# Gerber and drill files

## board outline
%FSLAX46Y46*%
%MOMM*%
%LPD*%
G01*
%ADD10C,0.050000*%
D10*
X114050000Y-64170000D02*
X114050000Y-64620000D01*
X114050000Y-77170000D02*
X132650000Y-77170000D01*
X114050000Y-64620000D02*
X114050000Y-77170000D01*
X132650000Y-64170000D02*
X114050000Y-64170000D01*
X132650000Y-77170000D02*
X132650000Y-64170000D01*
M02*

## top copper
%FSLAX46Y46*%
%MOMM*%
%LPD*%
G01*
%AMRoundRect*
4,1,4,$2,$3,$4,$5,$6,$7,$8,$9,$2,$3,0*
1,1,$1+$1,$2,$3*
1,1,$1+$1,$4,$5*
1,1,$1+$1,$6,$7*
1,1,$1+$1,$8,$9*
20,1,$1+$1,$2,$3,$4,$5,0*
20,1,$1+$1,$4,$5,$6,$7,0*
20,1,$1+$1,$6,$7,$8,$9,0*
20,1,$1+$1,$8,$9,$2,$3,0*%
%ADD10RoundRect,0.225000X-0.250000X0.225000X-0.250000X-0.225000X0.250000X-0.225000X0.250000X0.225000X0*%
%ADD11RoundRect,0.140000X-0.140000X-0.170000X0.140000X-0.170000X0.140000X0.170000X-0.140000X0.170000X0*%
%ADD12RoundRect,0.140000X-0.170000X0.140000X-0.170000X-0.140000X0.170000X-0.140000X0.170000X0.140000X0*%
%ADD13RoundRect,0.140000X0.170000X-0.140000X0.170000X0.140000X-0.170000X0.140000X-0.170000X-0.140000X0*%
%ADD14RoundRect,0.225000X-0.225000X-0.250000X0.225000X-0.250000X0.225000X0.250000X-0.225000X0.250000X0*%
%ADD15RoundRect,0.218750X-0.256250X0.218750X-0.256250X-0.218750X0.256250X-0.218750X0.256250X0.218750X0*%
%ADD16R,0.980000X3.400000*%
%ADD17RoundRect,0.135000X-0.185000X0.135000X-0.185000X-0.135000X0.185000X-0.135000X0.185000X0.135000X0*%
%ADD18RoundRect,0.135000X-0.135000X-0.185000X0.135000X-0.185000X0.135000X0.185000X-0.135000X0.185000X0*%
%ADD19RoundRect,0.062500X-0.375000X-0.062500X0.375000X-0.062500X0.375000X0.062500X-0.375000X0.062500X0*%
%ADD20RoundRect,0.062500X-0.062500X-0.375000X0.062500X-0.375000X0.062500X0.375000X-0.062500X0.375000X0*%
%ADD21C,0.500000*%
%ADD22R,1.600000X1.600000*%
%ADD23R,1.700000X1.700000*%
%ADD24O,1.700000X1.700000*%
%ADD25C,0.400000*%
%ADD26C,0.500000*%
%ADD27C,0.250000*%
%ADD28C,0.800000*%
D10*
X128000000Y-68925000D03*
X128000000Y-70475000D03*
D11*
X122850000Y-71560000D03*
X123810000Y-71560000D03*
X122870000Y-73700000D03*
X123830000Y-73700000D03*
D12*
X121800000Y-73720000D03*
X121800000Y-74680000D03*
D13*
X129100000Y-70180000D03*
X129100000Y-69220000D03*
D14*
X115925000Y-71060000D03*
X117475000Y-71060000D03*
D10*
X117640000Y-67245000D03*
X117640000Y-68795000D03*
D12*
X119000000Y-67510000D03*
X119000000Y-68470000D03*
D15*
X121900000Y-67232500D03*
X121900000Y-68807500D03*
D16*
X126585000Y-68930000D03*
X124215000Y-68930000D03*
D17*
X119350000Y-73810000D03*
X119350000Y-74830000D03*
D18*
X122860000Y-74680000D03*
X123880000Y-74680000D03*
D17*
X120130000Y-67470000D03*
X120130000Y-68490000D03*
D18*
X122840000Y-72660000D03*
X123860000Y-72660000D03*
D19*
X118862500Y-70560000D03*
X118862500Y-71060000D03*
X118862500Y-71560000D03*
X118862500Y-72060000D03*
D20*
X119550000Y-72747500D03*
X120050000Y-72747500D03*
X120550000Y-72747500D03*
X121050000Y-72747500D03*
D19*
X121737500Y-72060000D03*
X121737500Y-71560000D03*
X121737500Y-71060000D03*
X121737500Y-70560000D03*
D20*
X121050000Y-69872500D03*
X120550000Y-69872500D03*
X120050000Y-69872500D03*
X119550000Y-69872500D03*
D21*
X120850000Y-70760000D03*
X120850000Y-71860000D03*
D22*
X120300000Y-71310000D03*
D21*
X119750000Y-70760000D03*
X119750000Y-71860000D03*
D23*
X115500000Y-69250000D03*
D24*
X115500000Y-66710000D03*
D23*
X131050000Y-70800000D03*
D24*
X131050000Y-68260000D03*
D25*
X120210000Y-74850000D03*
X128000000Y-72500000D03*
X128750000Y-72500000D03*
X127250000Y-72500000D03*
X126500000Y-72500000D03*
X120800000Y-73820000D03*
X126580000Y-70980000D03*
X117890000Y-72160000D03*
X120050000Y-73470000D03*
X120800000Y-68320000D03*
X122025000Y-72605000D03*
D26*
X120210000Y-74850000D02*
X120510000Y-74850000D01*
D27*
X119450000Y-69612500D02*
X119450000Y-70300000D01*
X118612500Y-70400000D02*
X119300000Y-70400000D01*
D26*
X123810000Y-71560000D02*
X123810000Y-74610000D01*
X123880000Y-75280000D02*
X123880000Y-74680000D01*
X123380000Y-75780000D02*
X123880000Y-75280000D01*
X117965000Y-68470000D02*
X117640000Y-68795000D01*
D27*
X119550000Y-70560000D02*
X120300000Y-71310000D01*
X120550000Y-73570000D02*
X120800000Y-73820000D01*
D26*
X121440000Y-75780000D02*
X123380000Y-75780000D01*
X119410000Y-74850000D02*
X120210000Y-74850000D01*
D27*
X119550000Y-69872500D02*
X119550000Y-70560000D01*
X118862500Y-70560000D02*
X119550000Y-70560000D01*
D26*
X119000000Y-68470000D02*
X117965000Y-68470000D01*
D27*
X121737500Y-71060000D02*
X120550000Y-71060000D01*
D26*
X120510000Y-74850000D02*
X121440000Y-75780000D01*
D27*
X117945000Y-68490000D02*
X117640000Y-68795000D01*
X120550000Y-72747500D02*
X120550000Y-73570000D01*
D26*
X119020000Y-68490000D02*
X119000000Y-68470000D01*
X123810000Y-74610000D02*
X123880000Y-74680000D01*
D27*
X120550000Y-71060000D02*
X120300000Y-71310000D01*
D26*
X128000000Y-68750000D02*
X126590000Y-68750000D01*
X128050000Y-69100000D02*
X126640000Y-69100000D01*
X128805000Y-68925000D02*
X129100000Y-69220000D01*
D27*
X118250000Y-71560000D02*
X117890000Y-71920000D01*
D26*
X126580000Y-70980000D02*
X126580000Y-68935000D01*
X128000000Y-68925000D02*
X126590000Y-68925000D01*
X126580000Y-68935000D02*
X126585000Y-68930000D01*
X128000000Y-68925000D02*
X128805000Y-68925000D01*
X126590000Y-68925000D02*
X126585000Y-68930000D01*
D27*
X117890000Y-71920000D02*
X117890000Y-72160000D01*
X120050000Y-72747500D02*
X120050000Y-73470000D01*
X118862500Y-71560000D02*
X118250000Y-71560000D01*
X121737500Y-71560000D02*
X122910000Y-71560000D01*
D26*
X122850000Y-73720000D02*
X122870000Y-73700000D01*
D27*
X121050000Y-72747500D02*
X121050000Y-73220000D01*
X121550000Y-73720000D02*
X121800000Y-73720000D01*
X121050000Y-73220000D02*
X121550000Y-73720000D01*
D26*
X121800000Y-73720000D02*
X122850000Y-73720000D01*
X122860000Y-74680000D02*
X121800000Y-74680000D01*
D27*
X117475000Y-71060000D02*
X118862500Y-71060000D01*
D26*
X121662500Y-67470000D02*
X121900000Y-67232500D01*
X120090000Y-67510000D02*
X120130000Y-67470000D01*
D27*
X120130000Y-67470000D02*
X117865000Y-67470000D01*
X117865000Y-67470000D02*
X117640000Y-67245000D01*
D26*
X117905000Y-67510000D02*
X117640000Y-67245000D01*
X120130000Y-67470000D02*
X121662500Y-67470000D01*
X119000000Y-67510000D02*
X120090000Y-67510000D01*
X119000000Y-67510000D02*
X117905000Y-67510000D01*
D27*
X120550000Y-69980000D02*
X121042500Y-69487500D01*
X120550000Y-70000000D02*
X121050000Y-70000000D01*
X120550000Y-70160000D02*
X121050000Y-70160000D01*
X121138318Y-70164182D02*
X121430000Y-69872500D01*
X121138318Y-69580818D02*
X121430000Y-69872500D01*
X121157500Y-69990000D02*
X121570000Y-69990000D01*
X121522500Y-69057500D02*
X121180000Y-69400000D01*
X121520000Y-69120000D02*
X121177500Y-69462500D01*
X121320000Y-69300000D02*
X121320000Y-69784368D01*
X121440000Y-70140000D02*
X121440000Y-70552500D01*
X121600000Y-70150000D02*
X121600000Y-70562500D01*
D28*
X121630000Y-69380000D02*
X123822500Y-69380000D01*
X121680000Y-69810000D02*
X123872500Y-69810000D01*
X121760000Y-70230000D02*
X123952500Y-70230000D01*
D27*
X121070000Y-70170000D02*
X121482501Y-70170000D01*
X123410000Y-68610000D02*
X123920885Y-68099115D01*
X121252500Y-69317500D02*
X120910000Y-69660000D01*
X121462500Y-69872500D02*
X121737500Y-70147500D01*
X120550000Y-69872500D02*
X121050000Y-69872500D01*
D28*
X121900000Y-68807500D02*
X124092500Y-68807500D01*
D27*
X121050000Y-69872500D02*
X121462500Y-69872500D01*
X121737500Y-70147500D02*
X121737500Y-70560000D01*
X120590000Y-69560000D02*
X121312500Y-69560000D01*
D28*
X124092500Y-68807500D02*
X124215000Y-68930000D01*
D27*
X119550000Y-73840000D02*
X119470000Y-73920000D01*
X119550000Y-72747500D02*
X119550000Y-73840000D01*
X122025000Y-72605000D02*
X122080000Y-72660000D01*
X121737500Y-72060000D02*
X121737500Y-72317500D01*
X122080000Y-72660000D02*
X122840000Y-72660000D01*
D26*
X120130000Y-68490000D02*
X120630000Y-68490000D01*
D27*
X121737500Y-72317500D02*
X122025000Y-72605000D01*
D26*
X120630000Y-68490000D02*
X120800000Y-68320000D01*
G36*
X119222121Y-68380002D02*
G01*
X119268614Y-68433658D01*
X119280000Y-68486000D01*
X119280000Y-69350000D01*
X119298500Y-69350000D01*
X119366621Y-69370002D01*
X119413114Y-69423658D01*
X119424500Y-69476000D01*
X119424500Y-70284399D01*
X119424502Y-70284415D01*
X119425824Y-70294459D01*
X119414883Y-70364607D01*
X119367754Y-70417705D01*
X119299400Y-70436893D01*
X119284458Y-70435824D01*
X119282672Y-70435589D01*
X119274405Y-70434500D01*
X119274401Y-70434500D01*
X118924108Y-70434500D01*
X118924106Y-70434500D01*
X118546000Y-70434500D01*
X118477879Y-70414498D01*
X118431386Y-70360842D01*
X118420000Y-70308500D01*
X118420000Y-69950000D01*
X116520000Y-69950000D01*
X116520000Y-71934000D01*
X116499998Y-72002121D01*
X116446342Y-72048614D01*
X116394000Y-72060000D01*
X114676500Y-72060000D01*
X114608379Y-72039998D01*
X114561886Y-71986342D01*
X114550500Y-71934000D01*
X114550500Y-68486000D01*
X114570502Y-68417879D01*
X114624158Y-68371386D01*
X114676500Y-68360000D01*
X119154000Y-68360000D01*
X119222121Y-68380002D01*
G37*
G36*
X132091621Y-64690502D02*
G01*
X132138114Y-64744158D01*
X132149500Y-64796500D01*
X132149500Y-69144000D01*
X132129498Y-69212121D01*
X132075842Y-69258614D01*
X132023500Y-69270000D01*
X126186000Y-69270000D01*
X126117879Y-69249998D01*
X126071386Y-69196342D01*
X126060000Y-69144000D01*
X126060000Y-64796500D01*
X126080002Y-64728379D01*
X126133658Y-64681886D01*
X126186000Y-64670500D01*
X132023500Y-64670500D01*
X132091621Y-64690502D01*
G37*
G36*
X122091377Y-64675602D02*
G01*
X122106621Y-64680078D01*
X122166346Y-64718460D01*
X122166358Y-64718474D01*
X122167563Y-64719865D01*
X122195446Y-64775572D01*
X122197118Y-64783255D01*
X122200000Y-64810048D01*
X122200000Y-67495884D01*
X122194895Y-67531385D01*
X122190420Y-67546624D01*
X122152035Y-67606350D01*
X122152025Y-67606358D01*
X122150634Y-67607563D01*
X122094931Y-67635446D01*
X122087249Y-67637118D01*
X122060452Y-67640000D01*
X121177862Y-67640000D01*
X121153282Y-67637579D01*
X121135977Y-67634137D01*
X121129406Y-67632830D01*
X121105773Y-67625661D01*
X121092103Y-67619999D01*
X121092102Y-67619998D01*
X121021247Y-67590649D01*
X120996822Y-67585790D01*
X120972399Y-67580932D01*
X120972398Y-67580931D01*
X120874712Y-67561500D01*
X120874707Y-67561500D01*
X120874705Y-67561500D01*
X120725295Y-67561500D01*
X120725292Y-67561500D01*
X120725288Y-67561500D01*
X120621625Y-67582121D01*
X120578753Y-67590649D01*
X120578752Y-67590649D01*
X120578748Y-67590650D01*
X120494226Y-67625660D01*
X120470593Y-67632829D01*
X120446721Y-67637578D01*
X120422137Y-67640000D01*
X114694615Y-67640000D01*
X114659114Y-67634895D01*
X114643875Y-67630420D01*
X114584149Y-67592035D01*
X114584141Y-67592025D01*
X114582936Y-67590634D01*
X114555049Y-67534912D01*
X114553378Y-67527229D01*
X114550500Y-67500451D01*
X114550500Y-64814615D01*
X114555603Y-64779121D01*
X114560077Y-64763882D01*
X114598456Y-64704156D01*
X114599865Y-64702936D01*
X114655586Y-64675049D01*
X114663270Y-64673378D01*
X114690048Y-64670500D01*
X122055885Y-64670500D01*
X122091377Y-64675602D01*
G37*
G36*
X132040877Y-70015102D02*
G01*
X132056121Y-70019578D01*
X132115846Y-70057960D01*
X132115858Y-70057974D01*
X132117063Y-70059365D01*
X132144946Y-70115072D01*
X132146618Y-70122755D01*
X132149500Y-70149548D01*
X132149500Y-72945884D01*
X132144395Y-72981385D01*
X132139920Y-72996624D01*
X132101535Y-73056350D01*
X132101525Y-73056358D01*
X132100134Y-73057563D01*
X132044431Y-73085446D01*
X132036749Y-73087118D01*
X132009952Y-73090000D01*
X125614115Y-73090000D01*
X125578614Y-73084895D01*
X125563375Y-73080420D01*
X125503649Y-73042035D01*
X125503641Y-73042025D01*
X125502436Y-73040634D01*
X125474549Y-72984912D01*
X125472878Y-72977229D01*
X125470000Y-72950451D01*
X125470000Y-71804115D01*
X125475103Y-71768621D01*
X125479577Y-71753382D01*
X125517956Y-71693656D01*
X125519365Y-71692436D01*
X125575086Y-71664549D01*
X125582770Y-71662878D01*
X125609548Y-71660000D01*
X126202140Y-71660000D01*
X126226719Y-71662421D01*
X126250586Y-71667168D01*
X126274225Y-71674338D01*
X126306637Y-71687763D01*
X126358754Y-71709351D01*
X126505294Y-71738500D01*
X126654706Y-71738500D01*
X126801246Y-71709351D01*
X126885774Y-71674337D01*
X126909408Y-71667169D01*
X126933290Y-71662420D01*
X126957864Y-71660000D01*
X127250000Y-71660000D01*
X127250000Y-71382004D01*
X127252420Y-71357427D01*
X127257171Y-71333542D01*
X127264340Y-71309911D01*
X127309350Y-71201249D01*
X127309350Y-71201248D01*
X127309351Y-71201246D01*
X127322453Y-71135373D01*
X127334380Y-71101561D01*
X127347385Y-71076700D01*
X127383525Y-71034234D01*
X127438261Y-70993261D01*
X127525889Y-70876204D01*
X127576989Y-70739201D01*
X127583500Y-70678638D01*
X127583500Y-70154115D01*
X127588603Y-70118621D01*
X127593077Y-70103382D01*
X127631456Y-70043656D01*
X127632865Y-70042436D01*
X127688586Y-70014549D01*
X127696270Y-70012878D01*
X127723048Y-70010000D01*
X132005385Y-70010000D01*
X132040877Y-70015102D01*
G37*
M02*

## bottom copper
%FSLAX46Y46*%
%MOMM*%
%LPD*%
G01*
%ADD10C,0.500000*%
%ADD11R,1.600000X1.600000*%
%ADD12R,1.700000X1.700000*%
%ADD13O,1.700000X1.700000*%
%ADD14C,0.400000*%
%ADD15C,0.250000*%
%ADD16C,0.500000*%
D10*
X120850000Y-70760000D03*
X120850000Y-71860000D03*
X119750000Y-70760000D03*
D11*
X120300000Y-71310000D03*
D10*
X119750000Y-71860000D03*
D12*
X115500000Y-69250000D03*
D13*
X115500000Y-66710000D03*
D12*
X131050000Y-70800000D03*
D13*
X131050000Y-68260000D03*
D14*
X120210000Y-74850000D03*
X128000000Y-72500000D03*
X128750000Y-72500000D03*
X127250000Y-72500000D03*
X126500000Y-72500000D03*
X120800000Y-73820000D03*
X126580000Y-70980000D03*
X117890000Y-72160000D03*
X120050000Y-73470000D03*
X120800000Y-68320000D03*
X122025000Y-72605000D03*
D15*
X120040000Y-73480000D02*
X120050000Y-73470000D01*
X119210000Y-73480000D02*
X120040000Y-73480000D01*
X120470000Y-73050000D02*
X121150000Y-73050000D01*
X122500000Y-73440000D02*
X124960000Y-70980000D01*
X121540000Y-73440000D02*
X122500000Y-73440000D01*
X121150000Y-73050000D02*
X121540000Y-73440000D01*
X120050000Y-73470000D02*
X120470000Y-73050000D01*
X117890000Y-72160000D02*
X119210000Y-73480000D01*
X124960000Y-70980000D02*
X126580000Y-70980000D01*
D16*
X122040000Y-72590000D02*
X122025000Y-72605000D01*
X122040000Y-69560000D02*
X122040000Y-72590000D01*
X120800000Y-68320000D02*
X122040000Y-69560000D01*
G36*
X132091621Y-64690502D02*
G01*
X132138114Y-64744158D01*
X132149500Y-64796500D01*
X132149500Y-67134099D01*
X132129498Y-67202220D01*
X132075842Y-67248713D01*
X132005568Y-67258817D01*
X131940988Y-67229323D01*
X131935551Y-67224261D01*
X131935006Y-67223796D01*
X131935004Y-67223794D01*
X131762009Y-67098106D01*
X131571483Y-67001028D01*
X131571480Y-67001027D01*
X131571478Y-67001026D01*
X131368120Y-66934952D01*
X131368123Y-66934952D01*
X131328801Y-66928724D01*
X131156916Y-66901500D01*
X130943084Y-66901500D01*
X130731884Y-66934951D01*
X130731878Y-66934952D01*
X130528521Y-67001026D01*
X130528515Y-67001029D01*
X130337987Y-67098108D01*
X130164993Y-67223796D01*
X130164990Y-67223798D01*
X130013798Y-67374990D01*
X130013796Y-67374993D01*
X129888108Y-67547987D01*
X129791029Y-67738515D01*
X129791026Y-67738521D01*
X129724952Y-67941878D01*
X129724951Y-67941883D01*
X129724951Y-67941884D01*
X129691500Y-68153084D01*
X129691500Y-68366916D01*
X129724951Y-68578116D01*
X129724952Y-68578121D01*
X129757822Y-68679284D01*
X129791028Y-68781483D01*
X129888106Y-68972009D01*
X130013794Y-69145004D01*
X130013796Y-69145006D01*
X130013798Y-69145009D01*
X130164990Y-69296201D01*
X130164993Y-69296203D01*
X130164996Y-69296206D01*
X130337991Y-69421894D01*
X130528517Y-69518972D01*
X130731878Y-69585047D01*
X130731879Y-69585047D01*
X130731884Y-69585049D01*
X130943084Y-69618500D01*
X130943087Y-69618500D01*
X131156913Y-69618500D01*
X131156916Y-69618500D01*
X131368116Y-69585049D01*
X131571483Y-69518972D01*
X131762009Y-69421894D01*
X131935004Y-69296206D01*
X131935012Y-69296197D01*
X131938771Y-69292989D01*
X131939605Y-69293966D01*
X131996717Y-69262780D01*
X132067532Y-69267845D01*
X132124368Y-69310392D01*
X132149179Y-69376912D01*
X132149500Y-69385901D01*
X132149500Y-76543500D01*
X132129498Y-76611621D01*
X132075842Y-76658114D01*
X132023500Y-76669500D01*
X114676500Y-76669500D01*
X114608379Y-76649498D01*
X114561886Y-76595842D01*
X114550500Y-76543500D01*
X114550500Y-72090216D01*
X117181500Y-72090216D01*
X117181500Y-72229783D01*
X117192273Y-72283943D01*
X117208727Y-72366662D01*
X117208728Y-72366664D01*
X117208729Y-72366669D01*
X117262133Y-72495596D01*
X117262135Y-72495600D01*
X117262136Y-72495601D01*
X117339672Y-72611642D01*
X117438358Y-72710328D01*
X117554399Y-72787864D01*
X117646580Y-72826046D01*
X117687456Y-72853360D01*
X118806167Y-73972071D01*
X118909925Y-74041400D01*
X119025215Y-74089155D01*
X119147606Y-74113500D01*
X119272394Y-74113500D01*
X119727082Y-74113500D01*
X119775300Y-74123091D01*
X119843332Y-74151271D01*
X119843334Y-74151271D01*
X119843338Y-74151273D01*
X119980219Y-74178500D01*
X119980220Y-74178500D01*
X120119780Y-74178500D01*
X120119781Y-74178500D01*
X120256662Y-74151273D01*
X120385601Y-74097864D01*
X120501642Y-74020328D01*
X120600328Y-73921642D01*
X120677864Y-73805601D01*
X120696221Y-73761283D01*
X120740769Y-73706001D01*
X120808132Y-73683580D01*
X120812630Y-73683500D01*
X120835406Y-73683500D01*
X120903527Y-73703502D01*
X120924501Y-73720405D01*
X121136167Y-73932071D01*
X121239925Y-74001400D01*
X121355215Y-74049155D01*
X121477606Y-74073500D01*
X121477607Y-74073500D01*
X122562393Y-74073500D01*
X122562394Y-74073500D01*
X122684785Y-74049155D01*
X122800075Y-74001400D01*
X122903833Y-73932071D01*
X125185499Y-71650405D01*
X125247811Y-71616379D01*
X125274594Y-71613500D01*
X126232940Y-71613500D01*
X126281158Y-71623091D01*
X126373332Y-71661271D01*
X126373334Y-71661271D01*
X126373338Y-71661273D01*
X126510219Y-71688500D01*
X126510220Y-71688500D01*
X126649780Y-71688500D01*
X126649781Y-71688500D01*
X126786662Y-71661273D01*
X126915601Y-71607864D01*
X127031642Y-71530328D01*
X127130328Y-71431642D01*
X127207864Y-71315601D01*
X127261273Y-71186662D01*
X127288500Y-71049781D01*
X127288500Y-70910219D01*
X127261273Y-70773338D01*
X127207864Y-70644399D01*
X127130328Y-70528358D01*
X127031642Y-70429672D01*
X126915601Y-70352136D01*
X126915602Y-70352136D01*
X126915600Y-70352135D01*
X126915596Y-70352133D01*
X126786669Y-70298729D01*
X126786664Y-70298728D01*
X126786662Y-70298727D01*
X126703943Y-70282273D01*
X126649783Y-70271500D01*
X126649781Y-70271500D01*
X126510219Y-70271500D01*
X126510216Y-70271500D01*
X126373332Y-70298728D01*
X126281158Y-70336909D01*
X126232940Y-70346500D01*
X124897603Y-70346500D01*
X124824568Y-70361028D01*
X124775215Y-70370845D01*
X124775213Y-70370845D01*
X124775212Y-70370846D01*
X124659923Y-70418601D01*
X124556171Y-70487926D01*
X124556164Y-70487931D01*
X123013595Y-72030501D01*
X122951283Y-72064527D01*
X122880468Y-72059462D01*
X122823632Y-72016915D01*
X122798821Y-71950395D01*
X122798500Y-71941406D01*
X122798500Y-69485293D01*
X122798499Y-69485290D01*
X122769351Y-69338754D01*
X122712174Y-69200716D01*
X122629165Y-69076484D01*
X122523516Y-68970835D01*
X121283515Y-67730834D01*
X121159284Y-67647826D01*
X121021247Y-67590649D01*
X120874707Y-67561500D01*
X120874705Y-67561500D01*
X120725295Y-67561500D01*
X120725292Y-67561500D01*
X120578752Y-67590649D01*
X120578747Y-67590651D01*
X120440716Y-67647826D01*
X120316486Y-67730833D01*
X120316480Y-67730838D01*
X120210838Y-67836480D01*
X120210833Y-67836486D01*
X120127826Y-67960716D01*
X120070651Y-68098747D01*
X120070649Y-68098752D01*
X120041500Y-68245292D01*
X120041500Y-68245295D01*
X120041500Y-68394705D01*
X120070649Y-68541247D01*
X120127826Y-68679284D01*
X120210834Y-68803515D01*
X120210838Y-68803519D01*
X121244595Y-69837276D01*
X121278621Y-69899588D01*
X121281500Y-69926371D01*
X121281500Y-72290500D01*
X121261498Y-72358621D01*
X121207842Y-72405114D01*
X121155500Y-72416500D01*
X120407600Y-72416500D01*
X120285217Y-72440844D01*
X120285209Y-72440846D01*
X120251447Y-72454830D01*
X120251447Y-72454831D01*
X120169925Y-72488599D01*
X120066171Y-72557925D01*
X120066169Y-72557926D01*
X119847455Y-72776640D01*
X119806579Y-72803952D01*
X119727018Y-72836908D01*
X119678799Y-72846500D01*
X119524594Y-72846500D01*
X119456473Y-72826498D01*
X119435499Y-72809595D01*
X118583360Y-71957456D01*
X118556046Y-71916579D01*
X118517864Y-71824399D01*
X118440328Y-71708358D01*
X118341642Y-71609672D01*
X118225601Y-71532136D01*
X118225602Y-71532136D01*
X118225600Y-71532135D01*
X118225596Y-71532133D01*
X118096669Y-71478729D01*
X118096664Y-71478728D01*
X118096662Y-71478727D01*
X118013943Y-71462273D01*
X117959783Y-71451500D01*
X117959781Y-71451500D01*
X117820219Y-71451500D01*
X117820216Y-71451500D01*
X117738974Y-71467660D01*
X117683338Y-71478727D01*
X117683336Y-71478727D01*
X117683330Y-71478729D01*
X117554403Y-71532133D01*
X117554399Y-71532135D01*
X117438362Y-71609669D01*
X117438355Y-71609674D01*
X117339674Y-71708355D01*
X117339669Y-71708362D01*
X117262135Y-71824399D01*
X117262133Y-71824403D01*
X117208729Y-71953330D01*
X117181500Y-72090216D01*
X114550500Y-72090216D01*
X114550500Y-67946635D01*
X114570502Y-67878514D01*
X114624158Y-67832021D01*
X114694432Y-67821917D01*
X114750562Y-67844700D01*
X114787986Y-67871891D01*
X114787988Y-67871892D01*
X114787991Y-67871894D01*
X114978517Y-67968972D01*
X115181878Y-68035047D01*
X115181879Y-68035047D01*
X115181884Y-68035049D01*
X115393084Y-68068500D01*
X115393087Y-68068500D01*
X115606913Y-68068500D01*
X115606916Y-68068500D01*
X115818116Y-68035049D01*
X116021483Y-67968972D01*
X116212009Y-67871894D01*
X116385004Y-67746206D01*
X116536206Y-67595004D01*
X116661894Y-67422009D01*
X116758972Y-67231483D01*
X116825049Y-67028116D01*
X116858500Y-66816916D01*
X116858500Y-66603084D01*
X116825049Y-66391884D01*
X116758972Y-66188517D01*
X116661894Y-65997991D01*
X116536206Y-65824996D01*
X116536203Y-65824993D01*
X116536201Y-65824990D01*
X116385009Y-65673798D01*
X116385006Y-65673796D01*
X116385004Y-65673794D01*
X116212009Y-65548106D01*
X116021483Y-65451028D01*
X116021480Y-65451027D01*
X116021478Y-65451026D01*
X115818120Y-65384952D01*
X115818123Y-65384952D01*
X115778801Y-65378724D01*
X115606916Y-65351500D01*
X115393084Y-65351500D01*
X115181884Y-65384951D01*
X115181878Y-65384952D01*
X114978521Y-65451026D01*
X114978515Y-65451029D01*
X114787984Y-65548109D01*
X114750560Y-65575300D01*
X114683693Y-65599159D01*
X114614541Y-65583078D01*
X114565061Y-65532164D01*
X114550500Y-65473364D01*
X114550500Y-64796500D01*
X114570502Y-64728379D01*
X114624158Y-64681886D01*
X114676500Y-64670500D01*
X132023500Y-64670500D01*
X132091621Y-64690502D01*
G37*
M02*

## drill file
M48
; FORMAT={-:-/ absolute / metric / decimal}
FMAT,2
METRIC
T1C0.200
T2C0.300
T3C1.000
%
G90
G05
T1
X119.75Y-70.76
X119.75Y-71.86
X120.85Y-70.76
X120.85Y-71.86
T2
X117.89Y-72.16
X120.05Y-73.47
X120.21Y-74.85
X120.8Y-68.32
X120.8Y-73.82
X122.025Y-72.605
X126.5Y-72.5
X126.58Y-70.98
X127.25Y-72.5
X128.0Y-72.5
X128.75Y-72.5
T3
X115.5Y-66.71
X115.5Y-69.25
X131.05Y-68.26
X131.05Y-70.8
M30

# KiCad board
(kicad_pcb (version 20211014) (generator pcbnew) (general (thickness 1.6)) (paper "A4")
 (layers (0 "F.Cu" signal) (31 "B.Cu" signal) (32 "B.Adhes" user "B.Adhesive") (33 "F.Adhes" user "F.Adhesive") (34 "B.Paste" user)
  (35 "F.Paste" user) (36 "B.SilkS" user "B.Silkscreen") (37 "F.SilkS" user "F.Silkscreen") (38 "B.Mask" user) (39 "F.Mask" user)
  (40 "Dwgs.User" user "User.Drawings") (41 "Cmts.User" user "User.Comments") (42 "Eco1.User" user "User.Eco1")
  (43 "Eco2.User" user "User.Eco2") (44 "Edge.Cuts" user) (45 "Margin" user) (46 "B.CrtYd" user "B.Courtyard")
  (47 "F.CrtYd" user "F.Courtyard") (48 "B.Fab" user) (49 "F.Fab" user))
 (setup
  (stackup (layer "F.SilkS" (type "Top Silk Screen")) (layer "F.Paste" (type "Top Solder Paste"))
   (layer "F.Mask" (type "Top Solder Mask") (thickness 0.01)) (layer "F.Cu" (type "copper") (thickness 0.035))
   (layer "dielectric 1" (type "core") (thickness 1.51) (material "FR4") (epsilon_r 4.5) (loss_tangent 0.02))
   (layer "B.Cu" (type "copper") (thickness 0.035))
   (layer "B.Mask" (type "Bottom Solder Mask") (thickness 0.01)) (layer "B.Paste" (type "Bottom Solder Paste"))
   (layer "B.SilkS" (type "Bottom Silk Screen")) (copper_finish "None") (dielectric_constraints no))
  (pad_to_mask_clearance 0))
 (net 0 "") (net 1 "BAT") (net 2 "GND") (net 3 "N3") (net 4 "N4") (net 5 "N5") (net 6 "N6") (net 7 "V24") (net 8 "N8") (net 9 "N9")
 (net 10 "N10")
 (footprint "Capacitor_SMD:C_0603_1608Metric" (layer "F.Cu") (at 128 69.7 -90)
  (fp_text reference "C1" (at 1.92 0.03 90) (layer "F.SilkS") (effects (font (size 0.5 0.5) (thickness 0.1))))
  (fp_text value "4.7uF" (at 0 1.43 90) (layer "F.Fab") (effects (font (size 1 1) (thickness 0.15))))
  (pad "1" smd roundrect locked (at -0.775 0 270) (size 0.9 0.95) (layers "F.Cu" "F.Paste" "F.Mask") (roundrect_rratio 0.25) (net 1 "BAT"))
  (pad "2" smd roundrect locked (at 0.775 0 270) (size 0.9 0.95) (layers "F.Cu" "F.Paste" "F.Mask") (roundrect_rratio 0.25) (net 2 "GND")))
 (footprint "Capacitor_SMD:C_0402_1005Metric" (layer "F.Cu") (at 123.33 71.56)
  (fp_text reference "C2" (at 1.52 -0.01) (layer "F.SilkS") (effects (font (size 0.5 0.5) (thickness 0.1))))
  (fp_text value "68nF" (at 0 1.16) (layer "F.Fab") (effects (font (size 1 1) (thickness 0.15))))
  (pad "1" smd roundrect locked (at -0.48 0) (size 0.56 0.62) (layers "F.Cu" "F.Paste" "F.Mask") (roundrect_rratio 0.25) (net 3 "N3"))
  (pad "2" smd roundrect locked (at 0.48 0) (size 0.56 0.62) (layers "F.Cu" "F.Paste" "F.Mask") (roundrect_rratio 0.25) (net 2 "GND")))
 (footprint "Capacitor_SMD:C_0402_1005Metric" (layer "F.Cu") (at 123.35 73.7)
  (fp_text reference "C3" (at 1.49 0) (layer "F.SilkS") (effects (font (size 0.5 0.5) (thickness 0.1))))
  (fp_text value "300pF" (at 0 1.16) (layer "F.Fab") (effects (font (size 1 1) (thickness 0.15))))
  (pad "1" smd roundrect locked (at -0.48 0) (size 0.56 0.62) (layers "F.Cu" "F.Paste" "F.Mask") (roundrect_rratio 0.25) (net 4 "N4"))
  (pad "2" smd roundrect locked (at 0.48 0) (size 0.56 0.62) (layers "F.Cu" "F.Paste" "F.Mask") (roundrect_rratio 0.25) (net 2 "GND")))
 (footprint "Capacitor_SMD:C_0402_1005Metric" (layer "F.Cu") (at 121.8 74.2 -90)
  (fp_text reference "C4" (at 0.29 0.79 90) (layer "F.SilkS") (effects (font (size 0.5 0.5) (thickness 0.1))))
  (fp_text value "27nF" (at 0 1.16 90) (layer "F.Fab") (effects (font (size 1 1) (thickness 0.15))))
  (pad "1" smd roundrect locked (at -0.48 0 270) (size 0.56 0.62) (layers "F.Cu" "F.Paste" "F.Mask") (roundrect_rratio 0.25) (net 4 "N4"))
  (pad "2" smd roundrect locked (at 0.48 0 270) (size 0.56 0.62) (layers "F.Cu" "F.Paste" "F.Mask") (roundrect_rratio 0.25) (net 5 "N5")))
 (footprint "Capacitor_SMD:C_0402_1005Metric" (layer "F.Cu") (at 129.1 69.7 90)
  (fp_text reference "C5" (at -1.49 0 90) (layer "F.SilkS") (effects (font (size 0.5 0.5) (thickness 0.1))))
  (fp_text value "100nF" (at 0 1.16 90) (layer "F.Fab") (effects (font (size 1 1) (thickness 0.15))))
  (pad "1" smd roundrect locked (at -0.48 0 90) (size 0.56 0.62) (layers "F.Cu" "F.Paste" "F.Mask") (roundrect_rratio 0.25) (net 2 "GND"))
  (pad "2" smd roundrect locked (at 0.48 0 90) (size 0.56 0.62) (layers "F.Cu" "F.Paste" "F.Mask") (roundrect_rratio 0.25) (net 1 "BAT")))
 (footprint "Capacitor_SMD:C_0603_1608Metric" (layer "F.Cu") (at 116.7 71.06)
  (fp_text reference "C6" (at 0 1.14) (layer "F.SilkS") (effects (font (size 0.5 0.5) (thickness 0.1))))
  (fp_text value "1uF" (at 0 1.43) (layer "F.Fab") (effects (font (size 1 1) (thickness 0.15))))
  (pad "1" smd roundrect locked (at -0.775 0) (size 0.9 0.95) (layers "F.Cu" "F.Paste" "F.Mask") (roundrect_rratio 0.25) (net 2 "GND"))
  (pad "2" smd roundrect locked (at 0.775 0) (size 0.9 0.95) (layers "F.Cu" "F.Paste" "F.Mask") (roundrect_rratio 0.25) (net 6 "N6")))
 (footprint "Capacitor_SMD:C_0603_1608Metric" (layer "F.Cu") (at 117.64 68.02 -90)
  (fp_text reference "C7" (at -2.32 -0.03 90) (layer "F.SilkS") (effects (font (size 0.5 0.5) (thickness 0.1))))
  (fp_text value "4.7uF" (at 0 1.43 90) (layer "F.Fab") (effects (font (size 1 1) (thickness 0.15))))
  (pad "1" smd roundrect locked (at -0.775 0 270) (size 0.9 0.95) (layers "F.Cu" "F.Paste" "F.Mask") (roundrect_rratio 0.25) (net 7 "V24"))
  (pad "2" smd roundrect locked (at 0.775 0 270) (size 0.9 0.95) (layers "F.Cu" "F.Paste" "F.Mask") (roundrect_rratio 0.25) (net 2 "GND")))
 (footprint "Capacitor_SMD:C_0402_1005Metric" (layer "F.Cu") (at 119 67.99 -90)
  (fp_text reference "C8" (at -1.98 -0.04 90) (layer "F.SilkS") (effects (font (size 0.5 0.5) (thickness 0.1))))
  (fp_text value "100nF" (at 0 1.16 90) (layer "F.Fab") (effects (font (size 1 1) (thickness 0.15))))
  (pad "1" smd roundrect locked (at -0.48 0 270) (size 0.56 0.62) (layers "F.Cu" "F.Paste" "F.Mask") (roundrect_rratio 0.25) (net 7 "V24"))
  (pad "2" smd roundrect locked (at 0.48 0 270) (size 0.56 0.62) (layers "F.Cu" "F.Paste" "F.Mask") (roundrect_rratio 0.25) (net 2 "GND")))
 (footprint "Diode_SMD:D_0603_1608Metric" (layer "F.Cu") (at 121.9 68.02 -90)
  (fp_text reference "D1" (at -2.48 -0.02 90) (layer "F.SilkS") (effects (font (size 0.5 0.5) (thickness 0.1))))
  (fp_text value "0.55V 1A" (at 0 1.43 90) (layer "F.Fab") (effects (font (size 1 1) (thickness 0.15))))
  (pad "1" smd roundrect locked (at -0.7875 0 270) (size 0.875 0.95) (layers "F.Cu" "F.Paste" "F.Mask") (roundrect_rratio 0.25)
   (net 7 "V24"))
  (pad "2" smd roundrect locked (at 0.7875 0 270) (size 0.875 0.95) (layers "F.Cu" "F.Paste" "F.Mask") (roundrect_rratio 0.25) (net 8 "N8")))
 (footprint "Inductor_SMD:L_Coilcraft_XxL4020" (layer "F.Cu") (at 125.4 68.93 180)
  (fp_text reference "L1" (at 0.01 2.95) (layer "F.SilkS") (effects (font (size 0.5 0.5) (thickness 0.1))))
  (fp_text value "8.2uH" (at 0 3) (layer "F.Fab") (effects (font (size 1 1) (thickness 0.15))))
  (pad "1" smd rect locked (at -1.185 0 180) (size 0.98 3.4) (layers "F.Cu" "F.Paste" "F.Mask") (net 1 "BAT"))
  (pad "2" smd rect locked (at 1.185 0 180) (size 0.98 3.4) (layers "F.Cu" "F.Paste" "F.Mask") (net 8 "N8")))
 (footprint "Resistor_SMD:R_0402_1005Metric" (layer "F.Cu") (at 119.35 74.32 -90)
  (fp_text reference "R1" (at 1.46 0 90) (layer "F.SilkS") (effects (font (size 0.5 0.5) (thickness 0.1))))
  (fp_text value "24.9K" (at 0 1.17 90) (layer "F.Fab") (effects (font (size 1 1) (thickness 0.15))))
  (pad "1" smd roundrect locked (at -0.51 0 270) (size 0.54 0.64) (layers "F.Cu" "F.Paste" "F.Mask") (roundrect_rratio 0.25) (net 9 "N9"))
  (pad "2" smd roundrect locked (at 0.51 0 270) (size 0.54 0.64) (layers "F.Cu" "F.Paste" "F.Mask") (roundrect_rratio 0.25) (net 2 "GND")))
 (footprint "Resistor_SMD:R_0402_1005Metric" (layer "F.Cu") (at 123.37 74.68)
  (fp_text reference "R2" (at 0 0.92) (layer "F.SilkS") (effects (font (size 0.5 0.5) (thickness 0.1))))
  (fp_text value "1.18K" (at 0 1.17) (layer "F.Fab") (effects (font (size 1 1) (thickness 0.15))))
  (pad "1" smd roundrect locked (at -0.51 0) (size 0.54 0.64) (layers "F.Cu" "F.Paste" "F.Mask") (roundrect_rratio 0.25) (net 5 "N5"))
  (pad "2" smd roundrect locked (at 0.51 0) (size 0.54 0.64) (layers "F.Cu" "F.Paste" "F.Mask") (roundrect_rratio 0.25) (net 2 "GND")))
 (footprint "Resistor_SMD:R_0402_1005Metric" (layer "F.Cu") (at 120.13 67.98 -90)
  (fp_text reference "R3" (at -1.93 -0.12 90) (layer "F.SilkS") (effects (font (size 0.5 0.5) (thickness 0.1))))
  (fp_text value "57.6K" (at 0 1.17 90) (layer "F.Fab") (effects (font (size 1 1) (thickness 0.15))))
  (pad "1" smd roundrect locked (at -0.51 0 270) (size 0.54 0.64) (layers "F.Cu" "F.Paste" "F.Mask") (roundrect_rratio 0.25) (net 7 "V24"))
  (pad "2" smd roundrect locked (at 0.51 0 270) (size 0.54 0.64) (layers "F.Cu" "F.Paste" "F.Mask") (roundrect_rratio 0.25) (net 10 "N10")))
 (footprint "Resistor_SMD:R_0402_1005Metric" (layer "F.Cu") (at 123.35 72.66)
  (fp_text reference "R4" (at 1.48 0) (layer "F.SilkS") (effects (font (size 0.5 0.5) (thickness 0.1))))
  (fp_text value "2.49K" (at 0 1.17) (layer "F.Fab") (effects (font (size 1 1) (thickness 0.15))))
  (pad "1" smd roundrect locked (at -0.51 0) (size 0.54 0.64) (layers "F.Cu" "F.Paste" "F.Mask") (roundrect_rratio 0.25) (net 10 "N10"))
  (pad "2" smd roundrect locked (at 0.51 0) (size 0.54 0.64) (layers "F.Cu" "F.Paste" "F.Mask") (roundrect_rratio 0.25) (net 2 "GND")))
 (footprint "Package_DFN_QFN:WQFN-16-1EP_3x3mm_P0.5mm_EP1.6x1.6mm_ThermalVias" (layer "F.Cu") (at 120.3 71.31)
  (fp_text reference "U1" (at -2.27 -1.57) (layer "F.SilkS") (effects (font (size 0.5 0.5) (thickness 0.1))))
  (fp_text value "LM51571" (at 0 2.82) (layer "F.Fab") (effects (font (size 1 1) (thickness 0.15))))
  (pad "" smd roundrect locked (at 0.4 0.4) (size 0.69 0.69) (layers "F.Paste") (roundrect_rratio 0.25))
  (pad "" smd roundrect locked (at 0.4 -0.4) (size 0.69 0.69) (layers "F.Paste") (roundrect_rratio 0.25))
  (pad "" smd roundrect locked (at -0.4 0.4) (size 0.69 0.69) (layers "F.Paste") (roundrect_rratio 0.25))
  (pad "" smd roundrect locked (at -0.4 -0.4) (size 0.69 0.69) (layers "F.Paste") (roundrect_rratio 0.25))
  (pad "1" smd roundrect locked (at -1.4375 -0.75) (size 0.875 0.25) (layers "F.Cu" "F.Paste" "F.Mask") (roundrect_rratio 0.25)
   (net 2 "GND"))
  (pad "2" smd roundrect locked (at -1.4375 -0.25) (size 0.875 0.25) (layers "F.Cu" "F.Paste" "F.Mask") (roundrect_rratio 0.25) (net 6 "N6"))
  (pad "3" smd roundrect locked (at -1.4375 0.25) (size 0.875 0.25) (layers "F.Cu" "F.Paste" "F.Mask") (roundrect_rratio 0.25) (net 1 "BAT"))
  (pad "4" smd roundrect locked (at -1.4375 0.75) (size 0.875 0.25) (layers "F.Cu" "F.Paste" "F.Mask") (roundrect_rratio 0.25))
  (pad "5" smd roundrect locked (at -0.75 1.4375) (size 0.25 0.875) (layers "F.Cu" "F.Paste" "F.Mask") (roundrect_rratio 0.25) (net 9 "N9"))
  (pad "6" smd roundrect locked (at -0.25 1.4375) (size 0.25 0.875) (layers "F.Cu" "F.Paste" "F.Mask") (roundrect_rratio 0.25) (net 1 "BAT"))
  (pad "7" smd roundrect locked (at 0.25 1.4375) (size 0.25 0.875) (layers "F.Cu" "F.Paste" "F.Mask") (roundrect_rratio 0.25) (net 2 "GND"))
  (pad "8" smd roundrect locked (at 0.75 1.4375) (size 0.25 0.875) (layers "F.Cu" "F.Paste" "F.Mask") (roundrect_rratio 0.25) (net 4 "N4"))
  (pad "9" smd roundrect locked (at 1.4375 0.75) (size 0.875 0.25) (layers "F.Cu" "F.Paste" "F.Mask") (roundrect_rratio 0.25) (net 10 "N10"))
  (pad "10" smd roundrect locked (at 1.4375 0.25) (size 0.875 0.25) (layers "F.Cu" "F.Paste" "F.Mask") (roundrect_rratio 0.25) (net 3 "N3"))
  (pad "11" smd roundrect locked (at 1.4375 -0.25) (size 0.875 0.25) (layers "F.Cu" "F.Paste" "F.Mask") (roundrect_rratio 0.25)
   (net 2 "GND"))
  (pad "12" smd roundrect locked (at 1.4375 -0.75) (size 0.875 0.25) (layers "F.Cu" "F.Paste" "F.Mask") (roundrect_rratio 0.25) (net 8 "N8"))
  (pad "13" smd roundrect locked (at 0.75 -1.4375) (size 0.25 0.875) (layers "F.Cu" "F.Paste" "F.Mask") (roundrect_rratio 0.25) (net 8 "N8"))
  (pad "14" smd roundrect locked (at 0.25 -1.4375) (size 0.25 0.875) (layers "F.Cu" "F.Paste" "F.Mask") (roundrect_rratio 0.25) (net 8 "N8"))
  (pad "15" smd roundrect locked (at -0.25 -1.4375) (size 0.25 0.875) (layers "F.Cu" "F.Paste" "F.Mask") (roundrect_rratio 0.25))
  (pad "16" smd roundrect locked (at -0.75 -1.4375) (size 0.25 0.875) (layers "F.Cu" "F.Paste" "F.Mask") (roundrect_rratio 0.25)
   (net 2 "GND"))
  (pad "17" thru_hole circle locked (at 0.55 -0.55) (size 0.5 0.5) (drill 0.2) (layers *.Cu) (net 2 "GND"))
  (pad "17" thru_hole circle locked (at 0.55 0.55) (size 0.5 0.5) (drill 0.2) (layers *.Cu) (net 2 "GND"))
  (pad "17" smd rect locked (at 0 0) (size 1.6 1.6) (layers "F.Cu" "F.Mask") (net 2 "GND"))
  (pad "17" thru_hole circle locked (at -0.55 -0.55) (size 0.5 0.5) (drill 0.2) (layers *.Cu) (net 2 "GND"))
  (pad "17" smd rect locked (at 0 0) (size 1.6 1.6) (layers "B.Cu") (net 2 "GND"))
  (pad "17" thru_hole circle locked (at -0.55 0.55) (size 0.5 0.5) (drill 0.2) (layers *.Cu) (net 2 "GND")))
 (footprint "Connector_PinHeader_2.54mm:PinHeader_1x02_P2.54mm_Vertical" (layer "F.Cu") (at 115.5 69.25 180)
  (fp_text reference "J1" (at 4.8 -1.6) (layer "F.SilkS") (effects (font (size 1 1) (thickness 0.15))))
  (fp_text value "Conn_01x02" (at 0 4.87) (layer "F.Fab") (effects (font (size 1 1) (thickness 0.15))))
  (pad "1" thru_hole rect locked (at 0 0 180) (size 1.7 1.7) (drill 1) (layers *.Cu *.Mask) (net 2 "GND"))
  (pad "2" thru_hole oval locked (at 0 2.54 180) (size 1.7 1.7) (drill 1) (layers *.Cu *.Mask) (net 7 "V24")))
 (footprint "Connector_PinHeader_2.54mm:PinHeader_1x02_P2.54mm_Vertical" (layer "F.Cu") (at 131.05 70.8 180)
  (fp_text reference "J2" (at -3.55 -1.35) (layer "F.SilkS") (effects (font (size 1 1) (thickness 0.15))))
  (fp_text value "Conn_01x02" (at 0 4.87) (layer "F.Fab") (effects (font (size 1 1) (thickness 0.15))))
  (pad "1" thru_hole rect locked (at 0 0 180) (size 1.7 1.7) (drill 1) (layers *.Cu *.Mask) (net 2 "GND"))
  (pad "2" thru_hole oval locked (at 0 2.54 180) (size 1.7 1.7) (drill 1) (layers *.Cu *.Mask) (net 1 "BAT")))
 (gr_line (start 114.05 64.17) (end 114.05 64.62) (layer "Edge.Cuts") (width 0.05))
 (gr_line (start 114.05 77.17) (end 132.65 77.17) (layer "Edge.Cuts") (width 0.05))
 (gr_line (start 114.05 64.62) (end 114.05 77.17) (layer "Edge.Cuts") (width 0.05))
 (gr_line (start 132.65 64.17) (end 114.05 64.17) (layer "Edge.Cuts") (width 0.05))
 (gr_line (start 132.65 77.17) (end 132.65 64.17) (layer "Edge.Cuts") (width 0.05))
 (segment (start 120.21 74.85) (end 120.51 74.85) (width 0.5) (layer "F.Cu") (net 2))
 (segment (start 119.45 69.6125) (end 119.45 70.3) (width 0.25) (layer "F.Cu") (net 2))
 (segment (start 118.6125 70.4) (end 119.3 70.4) (width 0.25) (layer "F.Cu") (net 2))
 (segment (start 123.81 71.56) (end 123.81 74.61) (width 0.5) (layer "F.Cu") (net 2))
 (segment (start 123.88 75.28) (end 123.88 74.68) (width 0.5) (layer "F.Cu") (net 2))
 (segment (start 123.38 75.78) (end 123.88 75.28) (width 0.5) (layer "F.Cu") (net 2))
 (segment (start 117.965 68.47) (end 117.64 68.795) (width 0.5) (layer "F.Cu") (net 2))
 (segment (start 119.55 70.56) (end 120.3 71.31) (width 0.25) (layer "F.Cu") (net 2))
 (segment (start 120.55 73.57) (end 120.8 73.82) (width 0.25) (layer "F.Cu") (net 2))
 (segment (start 121.44 75.78) (end 123.38 75.78) (width 0.5) (layer "F.Cu") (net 2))
 (segment (start 119.41 74.85) (end 120.21 74.85) (width 0.5) (layer "F.Cu") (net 2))
 (segment (start 119.55 69.8725) (end 119.55 70.56) (width 0.25) (layer "F.Cu") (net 2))
 (segment (start 118.8625 70.56) (end 119.55 70.56) (width 0.25) (layer "F.Cu") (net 2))
 (segment (start 119 68.47) (end 117.965 68.47) (width 0.5) (layer "F.Cu") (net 2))
 (segment (start 121.7375 71.06) (end 120.55 71.06) (width 0.25) (layer "F.Cu") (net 2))
 (segment (start 120.51 74.85) (end 121.44 75.78) (width 0.5) (layer "F.Cu") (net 2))
 (segment (start 117.945 68.49) (end 117.64 68.795) (width 0.25) (layer "F.Cu") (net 2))
 (segment (start 120.55 72.7475) (end 120.55 73.57) (width 0.25) (layer "F.Cu") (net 2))
 (segment (start 119.02 68.49) (end 119 68.47) (width 0.5) (layer "F.Cu") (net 2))
 (segment (start 123.81 74.61) (end 123.88 74.68) (width 0.5) (layer "F.Cu") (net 2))
 (segment (start 120.55 71.06) (end 120.3 71.31) (width 0.25) (layer "F.Cu") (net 2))
 (via (at 120.21 74.85) (size 0.4) (drill 0.3) (layers "F.Cu" "B.Cu") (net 2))
 (via (at 128 72.5) (size 0.4) (drill 0.3) (layers "F.Cu" "B.Cu") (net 2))
 (via (at 128.75 72.5) (size 0.4) (drill 0.3) (layers "F.Cu" "B.Cu") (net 2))
 (via (at 127.25 72.5) (size 0.4) (drill 0.3) (layers "F.Cu" "B.Cu") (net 2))
 (via (at 126.5 72.5) (size 0.4) (drill 0.3) (layers "F.Cu" "B.Cu") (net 2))
 (via (at 120.8 73.82) (size 0.4) (drill 0.3) (layers "F.Cu" "B.Cu") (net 2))
 (segment (start 128 68.75) (end 126.59 68.75) (width 0.5) (layer "F.Cu") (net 1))
 (segment (start 128.05 69.1) (end 126.64 69.1) (width 0.5) (layer "F.Cu") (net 1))
 (segment (start 128.805 68.925) (end 129.1 69.22) (width 0.5) (layer "F.Cu") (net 1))
 (segment (start 118.25 71.56) (end 117.89 71.92) (width 0.25) (layer "F.Cu") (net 1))
 (segment (start 126.58 70.98) (end 126.58 68.935) (width 0.5) (layer "F.Cu") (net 1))
 (segment (start 128 68.925) (end 126.59 68.925) (width 0.5) (layer "F.Cu") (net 1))
 (segment (start 126.58 68.935) (end 126.585 68.93) (width 0.5) (layer "F.Cu") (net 1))
 (segment (start 128 68.925) (end 128.805 68.925) (width 0.5) (layer "F.Cu") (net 1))
 (segment (start 126.59 68.925) (end 126.585 68.93) (width 0.5) (layer "F.Cu") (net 1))
 (segment (start 117.89 71.92) (end 117.89 72.16) (width 0.25) (layer "F.Cu") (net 1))
 (segment (start 120.05 72.7475) (end 120.05 73.47) (width 0.25) (layer "F.Cu") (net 1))
 (segment (start 118.8625 71.56) (end 118.25 71.56) (width 0.25) (layer "F.Cu") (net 1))
 (via (at 126.58 70.98) (size 0.4) (drill 0.3) (layers "F.Cu" "B.Cu") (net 1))
 (via (at 117.89 72.16) (size 0.4) (drill 0.3) (layers "F.Cu" "B.Cu") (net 1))
 (via (at 120.05 73.47) (size 0.4) (drill 0.3) (layers "F.Cu" "B.Cu") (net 1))
 (segment (start 120.04 73.48) (end 120.05 73.47) (width 0.25) (layer "B.Cu") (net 1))
 (segment (start 119.21 73.48) (end 120.04 73.48) (width 0.25) (layer "B.Cu") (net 1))
 (segment (start 120.47 73.05) (end 121.15 73.05) (width 0.25) (layer "B.Cu") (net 1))
 (segment (start 122.5 73.44) (end 124.96 70.98) (width 0.25) (layer "B.Cu") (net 1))
 (segment (start 121.54 73.44) (end 122.5 73.44) (width 0.25) (layer "B.Cu") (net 1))
 (segment (start 121.15 73.05) (end 121.54 73.44) (width 0.25) (layer "B.Cu") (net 1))
 (segment (start 120.05 73.47) (end 120.47 73.05) (width 0.25) (layer "B.Cu") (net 1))
 (segment (start 117.89 72.16) (end 119.21 73.48) (width 0.25) (layer "B.Cu") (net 1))
 (segment (start 124.96 70.98) (end 126.58 70.98) (width 0.25) (layer "B.Cu") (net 1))
 (segment (start 121.7375 71.56) (end 122.91 71.56) (width 0.25) (layer "F.Cu") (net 3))
 (segment (start 122.85 73.72) (end 122.87 73.7) (width 0.5) (layer "F.Cu") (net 4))
 (segment (start 121.05 72.7475) (end 121.05 73.22) (width 0.25) (layer "F.Cu") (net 4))
 (segment (start 121.55 73.72) (end 121.8 73.72) (width 0.25) (layer "F.Cu") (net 4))
 (segment (start 121.05 73.22) (end 121.55 73.72) (width 0.25) (layer "F.Cu") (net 4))
 (segment (start 121.8 73.72) (end 122.85 73.72) (width 0.5) (layer "F.Cu") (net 4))
 (segment (start 122.86 74.68) (end 121.8 74.68) (width 0.5) (layer "F.Cu") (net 5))
 (segment (start 117.475 71.06) (end 118.8625 71.06) (width 0.25) (layer "F.Cu") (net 6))
 (segment (start 121.6625 67.47) (end 121.9 67.2325) (width 0.5) (layer "F.Cu") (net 7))
 (segment (start 120.09 67.51) (end 120.13 67.47) (width 0.5) (layer "F.Cu") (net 7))
 (segment (start 120.13 67.47) (end 117.865 67.47) (width 0.25) (layer "F.Cu") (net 7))
 (segment (start 117.865 67.47) (end 117.64 67.245) (width 0.25) (layer "F.Cu") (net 7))
 (segment (start 117.905 67.51) (end 117.64 67.245) (width 0.5) (layer "F.Cu") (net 7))
 (segment (start 120.13 67.47) (end 121.6625 67.47) (width 0.5) (layer "F.Cu") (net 7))
 (segment (start 119 67.51) (end 120.09 67.51) (width 0.5) (layer "F.Cu") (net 7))
 (segment (start 119 67.51) (end 117.905 67.51) (width 0.5) (layer "F.Cu") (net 7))
 (segment (start 120.55 69.98) (end 121.0425 69.4875) (width 0.25) (layer "F.Cu") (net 8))
 (segment (start 120.55 70) (end 121.05 70) (width 0.25) (layer "F.Cu") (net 8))
 (segment (start 120.55 70.16) (end 121.05 70.16) (width 0.25) (layer "F.Cu") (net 8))
 (segment (start 121.138318 70.164182) (end 121.43 69.8725) (width 0.25) (layer "F.Cu") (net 8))
 (segment (start 121.138318 69.580818) (end 121.43 69.8725) (width 0.25) (layer "F.Cu") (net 8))
 (segment (start 121.1575 69.99) (end 121.57 69.99) (width 0.25) (layer "F.Cu") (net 8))
 (segment (start 121.5225 69.0575) (end 121.18 69.4) (width 0.25) (layer "F.Cu") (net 8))
 (segment (start 121.52 69.12) (end 121.1775 69.4625) (width 0.25) (layer "F.Cu") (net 8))
 (segment (start 121.32 69.3) (end 121.32 69.784368) (width 0.25) (layer "F.Cu") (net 8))
 (segment (start 121.44 70.14) (end 121.44 70.5525) (width 0.25) (layer "F.Cu") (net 8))
 (segment (start 121.6 70.15) (end 121.6 70.5625) (width 0.25) (layer "F.Cu") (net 8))
 (segment (start 121.63 69.38) (end 123.8225 69.38) (width 0.8) (layer "F.Cu") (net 8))
 (segment (start 121.68 69.81) (end 123.8725 69.81) (width 0.8) (layer "F.Cu") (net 8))
 (segment (start 121.76 70.23) (end 123.9525 70.23) (width 0.8) (layer "F.Cu") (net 8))
 (segment (start 121.07 70.17) (end 121.482501 70.17) (width 0.25) (layer "F.Cu") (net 8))
 (segment (start 123.41 68.61) (end 123.920885 68.099115) (width 0.25) (layer "F.Cu") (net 8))
 (segment (start 121.2525 69.3175) (end 120.91 69.66) (width 0.25) (layer "F.Cu") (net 8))
 (segment (start 121.4625 69.8725) (end 121.7375 70.1475) (width 0.25) (layer "F.Cu") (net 8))
 (segment (start 120.55 69.8725) (end 121.05 69.8725) (width 0.25) (layer "F.Cu") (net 8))
 (segment (start 121.9 68.8075) (end 124.0925 68.8075) (width 0.8) (layer "F.Cu") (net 8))
 (segment (start 121.05 69.8725) (end 121.4625 69.8725) (width 0.25) (layer "F.Cu") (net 8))
 (segment (start 121.7375 70.1475) (end 121.7375 70.56) (width 0.25) (layer "F.Cu") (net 8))
 (segment (start 120.59 69.56) (end 121.3125 69.56) (width 0.25) (layer "F.Cu") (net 8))
 (segment (start 124.0925 68.8075) (end 124.215 68.93) (width 0.8) (layer "F.Cu") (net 8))
 (segment (start 119.55 73.84) (end 119.47 73.92) (width 0.25) (layer "F.Cu") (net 9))
 (segment (start 119.55 72.7475) (end 119.55 73.84) (width 0.25) (layer "F.Cu") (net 9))
 (segment (start 122.025 72.605) (end 122.08 72.66) (width 0.25) (layer "F.Cu") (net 10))
 (segment (start 121.7375 72.06) (end 121.7375 72.3175) (width 0.25) (layer "F.Cu") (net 10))
 (segment (start 122.08 72.66) (end 122.84 72.66) (width 0.25) (layer "F.Cu") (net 10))
 (segment (start 120.13 68.49) (end 120.63 68.49) (width 0.5) (layer "F.Cu") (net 10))
 (segment (start 121.7375 72.3175) (end 122.025 72.605) (width 0.25) (layer "F.Cu") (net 10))
 (segment (start 120.63 68.49) (end 120.8 68.32) (width 0.5) (layer "F.Cu") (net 10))
 (via (at 120.8 68.32) (size 0.4) (drill 0.3) (layers "F.Cu" "B.Cu") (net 10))
 (via (at 122.025 72.605) (size 0.4) (drill 0.3) (layers "F.Cu" "B.Cu") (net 10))
 (segment (start 122.04 72.59) (end 122.025 72.605) (width 0.5) (layer "B.Cu") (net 10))
 (segment (start 122.04 69.56) (end 122.04 72.59) (width 0.5) (layer "B.Cu") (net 10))
 (segment (start 120.8 68.32) (end 122.04 69.56) (width 0.5) (layer "B.Cu") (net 10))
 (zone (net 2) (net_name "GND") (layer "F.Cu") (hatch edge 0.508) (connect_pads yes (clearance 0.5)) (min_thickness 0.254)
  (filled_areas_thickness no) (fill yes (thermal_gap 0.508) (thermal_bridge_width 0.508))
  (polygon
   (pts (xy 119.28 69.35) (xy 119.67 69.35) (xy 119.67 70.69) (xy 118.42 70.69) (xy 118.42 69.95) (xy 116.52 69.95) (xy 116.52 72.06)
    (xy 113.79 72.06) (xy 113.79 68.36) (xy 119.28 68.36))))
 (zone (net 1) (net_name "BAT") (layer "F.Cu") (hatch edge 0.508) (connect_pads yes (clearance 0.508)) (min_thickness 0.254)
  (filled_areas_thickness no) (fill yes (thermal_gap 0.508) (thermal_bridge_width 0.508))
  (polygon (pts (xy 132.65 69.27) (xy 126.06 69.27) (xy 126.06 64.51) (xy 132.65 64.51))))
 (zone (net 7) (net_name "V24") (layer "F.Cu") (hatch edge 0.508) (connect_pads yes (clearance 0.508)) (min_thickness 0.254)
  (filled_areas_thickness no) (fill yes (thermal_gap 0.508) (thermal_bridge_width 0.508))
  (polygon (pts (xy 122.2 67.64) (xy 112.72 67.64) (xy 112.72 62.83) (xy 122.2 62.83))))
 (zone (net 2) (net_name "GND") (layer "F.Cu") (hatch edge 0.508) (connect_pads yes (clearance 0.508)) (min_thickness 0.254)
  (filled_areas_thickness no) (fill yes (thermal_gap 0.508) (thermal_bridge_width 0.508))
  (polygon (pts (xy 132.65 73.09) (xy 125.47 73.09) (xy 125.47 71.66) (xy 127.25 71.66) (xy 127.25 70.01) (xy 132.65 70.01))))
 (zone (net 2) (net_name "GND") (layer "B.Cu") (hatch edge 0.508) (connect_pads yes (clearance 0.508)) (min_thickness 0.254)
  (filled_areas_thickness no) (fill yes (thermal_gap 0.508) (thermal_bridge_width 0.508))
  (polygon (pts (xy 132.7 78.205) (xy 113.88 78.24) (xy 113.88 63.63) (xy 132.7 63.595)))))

